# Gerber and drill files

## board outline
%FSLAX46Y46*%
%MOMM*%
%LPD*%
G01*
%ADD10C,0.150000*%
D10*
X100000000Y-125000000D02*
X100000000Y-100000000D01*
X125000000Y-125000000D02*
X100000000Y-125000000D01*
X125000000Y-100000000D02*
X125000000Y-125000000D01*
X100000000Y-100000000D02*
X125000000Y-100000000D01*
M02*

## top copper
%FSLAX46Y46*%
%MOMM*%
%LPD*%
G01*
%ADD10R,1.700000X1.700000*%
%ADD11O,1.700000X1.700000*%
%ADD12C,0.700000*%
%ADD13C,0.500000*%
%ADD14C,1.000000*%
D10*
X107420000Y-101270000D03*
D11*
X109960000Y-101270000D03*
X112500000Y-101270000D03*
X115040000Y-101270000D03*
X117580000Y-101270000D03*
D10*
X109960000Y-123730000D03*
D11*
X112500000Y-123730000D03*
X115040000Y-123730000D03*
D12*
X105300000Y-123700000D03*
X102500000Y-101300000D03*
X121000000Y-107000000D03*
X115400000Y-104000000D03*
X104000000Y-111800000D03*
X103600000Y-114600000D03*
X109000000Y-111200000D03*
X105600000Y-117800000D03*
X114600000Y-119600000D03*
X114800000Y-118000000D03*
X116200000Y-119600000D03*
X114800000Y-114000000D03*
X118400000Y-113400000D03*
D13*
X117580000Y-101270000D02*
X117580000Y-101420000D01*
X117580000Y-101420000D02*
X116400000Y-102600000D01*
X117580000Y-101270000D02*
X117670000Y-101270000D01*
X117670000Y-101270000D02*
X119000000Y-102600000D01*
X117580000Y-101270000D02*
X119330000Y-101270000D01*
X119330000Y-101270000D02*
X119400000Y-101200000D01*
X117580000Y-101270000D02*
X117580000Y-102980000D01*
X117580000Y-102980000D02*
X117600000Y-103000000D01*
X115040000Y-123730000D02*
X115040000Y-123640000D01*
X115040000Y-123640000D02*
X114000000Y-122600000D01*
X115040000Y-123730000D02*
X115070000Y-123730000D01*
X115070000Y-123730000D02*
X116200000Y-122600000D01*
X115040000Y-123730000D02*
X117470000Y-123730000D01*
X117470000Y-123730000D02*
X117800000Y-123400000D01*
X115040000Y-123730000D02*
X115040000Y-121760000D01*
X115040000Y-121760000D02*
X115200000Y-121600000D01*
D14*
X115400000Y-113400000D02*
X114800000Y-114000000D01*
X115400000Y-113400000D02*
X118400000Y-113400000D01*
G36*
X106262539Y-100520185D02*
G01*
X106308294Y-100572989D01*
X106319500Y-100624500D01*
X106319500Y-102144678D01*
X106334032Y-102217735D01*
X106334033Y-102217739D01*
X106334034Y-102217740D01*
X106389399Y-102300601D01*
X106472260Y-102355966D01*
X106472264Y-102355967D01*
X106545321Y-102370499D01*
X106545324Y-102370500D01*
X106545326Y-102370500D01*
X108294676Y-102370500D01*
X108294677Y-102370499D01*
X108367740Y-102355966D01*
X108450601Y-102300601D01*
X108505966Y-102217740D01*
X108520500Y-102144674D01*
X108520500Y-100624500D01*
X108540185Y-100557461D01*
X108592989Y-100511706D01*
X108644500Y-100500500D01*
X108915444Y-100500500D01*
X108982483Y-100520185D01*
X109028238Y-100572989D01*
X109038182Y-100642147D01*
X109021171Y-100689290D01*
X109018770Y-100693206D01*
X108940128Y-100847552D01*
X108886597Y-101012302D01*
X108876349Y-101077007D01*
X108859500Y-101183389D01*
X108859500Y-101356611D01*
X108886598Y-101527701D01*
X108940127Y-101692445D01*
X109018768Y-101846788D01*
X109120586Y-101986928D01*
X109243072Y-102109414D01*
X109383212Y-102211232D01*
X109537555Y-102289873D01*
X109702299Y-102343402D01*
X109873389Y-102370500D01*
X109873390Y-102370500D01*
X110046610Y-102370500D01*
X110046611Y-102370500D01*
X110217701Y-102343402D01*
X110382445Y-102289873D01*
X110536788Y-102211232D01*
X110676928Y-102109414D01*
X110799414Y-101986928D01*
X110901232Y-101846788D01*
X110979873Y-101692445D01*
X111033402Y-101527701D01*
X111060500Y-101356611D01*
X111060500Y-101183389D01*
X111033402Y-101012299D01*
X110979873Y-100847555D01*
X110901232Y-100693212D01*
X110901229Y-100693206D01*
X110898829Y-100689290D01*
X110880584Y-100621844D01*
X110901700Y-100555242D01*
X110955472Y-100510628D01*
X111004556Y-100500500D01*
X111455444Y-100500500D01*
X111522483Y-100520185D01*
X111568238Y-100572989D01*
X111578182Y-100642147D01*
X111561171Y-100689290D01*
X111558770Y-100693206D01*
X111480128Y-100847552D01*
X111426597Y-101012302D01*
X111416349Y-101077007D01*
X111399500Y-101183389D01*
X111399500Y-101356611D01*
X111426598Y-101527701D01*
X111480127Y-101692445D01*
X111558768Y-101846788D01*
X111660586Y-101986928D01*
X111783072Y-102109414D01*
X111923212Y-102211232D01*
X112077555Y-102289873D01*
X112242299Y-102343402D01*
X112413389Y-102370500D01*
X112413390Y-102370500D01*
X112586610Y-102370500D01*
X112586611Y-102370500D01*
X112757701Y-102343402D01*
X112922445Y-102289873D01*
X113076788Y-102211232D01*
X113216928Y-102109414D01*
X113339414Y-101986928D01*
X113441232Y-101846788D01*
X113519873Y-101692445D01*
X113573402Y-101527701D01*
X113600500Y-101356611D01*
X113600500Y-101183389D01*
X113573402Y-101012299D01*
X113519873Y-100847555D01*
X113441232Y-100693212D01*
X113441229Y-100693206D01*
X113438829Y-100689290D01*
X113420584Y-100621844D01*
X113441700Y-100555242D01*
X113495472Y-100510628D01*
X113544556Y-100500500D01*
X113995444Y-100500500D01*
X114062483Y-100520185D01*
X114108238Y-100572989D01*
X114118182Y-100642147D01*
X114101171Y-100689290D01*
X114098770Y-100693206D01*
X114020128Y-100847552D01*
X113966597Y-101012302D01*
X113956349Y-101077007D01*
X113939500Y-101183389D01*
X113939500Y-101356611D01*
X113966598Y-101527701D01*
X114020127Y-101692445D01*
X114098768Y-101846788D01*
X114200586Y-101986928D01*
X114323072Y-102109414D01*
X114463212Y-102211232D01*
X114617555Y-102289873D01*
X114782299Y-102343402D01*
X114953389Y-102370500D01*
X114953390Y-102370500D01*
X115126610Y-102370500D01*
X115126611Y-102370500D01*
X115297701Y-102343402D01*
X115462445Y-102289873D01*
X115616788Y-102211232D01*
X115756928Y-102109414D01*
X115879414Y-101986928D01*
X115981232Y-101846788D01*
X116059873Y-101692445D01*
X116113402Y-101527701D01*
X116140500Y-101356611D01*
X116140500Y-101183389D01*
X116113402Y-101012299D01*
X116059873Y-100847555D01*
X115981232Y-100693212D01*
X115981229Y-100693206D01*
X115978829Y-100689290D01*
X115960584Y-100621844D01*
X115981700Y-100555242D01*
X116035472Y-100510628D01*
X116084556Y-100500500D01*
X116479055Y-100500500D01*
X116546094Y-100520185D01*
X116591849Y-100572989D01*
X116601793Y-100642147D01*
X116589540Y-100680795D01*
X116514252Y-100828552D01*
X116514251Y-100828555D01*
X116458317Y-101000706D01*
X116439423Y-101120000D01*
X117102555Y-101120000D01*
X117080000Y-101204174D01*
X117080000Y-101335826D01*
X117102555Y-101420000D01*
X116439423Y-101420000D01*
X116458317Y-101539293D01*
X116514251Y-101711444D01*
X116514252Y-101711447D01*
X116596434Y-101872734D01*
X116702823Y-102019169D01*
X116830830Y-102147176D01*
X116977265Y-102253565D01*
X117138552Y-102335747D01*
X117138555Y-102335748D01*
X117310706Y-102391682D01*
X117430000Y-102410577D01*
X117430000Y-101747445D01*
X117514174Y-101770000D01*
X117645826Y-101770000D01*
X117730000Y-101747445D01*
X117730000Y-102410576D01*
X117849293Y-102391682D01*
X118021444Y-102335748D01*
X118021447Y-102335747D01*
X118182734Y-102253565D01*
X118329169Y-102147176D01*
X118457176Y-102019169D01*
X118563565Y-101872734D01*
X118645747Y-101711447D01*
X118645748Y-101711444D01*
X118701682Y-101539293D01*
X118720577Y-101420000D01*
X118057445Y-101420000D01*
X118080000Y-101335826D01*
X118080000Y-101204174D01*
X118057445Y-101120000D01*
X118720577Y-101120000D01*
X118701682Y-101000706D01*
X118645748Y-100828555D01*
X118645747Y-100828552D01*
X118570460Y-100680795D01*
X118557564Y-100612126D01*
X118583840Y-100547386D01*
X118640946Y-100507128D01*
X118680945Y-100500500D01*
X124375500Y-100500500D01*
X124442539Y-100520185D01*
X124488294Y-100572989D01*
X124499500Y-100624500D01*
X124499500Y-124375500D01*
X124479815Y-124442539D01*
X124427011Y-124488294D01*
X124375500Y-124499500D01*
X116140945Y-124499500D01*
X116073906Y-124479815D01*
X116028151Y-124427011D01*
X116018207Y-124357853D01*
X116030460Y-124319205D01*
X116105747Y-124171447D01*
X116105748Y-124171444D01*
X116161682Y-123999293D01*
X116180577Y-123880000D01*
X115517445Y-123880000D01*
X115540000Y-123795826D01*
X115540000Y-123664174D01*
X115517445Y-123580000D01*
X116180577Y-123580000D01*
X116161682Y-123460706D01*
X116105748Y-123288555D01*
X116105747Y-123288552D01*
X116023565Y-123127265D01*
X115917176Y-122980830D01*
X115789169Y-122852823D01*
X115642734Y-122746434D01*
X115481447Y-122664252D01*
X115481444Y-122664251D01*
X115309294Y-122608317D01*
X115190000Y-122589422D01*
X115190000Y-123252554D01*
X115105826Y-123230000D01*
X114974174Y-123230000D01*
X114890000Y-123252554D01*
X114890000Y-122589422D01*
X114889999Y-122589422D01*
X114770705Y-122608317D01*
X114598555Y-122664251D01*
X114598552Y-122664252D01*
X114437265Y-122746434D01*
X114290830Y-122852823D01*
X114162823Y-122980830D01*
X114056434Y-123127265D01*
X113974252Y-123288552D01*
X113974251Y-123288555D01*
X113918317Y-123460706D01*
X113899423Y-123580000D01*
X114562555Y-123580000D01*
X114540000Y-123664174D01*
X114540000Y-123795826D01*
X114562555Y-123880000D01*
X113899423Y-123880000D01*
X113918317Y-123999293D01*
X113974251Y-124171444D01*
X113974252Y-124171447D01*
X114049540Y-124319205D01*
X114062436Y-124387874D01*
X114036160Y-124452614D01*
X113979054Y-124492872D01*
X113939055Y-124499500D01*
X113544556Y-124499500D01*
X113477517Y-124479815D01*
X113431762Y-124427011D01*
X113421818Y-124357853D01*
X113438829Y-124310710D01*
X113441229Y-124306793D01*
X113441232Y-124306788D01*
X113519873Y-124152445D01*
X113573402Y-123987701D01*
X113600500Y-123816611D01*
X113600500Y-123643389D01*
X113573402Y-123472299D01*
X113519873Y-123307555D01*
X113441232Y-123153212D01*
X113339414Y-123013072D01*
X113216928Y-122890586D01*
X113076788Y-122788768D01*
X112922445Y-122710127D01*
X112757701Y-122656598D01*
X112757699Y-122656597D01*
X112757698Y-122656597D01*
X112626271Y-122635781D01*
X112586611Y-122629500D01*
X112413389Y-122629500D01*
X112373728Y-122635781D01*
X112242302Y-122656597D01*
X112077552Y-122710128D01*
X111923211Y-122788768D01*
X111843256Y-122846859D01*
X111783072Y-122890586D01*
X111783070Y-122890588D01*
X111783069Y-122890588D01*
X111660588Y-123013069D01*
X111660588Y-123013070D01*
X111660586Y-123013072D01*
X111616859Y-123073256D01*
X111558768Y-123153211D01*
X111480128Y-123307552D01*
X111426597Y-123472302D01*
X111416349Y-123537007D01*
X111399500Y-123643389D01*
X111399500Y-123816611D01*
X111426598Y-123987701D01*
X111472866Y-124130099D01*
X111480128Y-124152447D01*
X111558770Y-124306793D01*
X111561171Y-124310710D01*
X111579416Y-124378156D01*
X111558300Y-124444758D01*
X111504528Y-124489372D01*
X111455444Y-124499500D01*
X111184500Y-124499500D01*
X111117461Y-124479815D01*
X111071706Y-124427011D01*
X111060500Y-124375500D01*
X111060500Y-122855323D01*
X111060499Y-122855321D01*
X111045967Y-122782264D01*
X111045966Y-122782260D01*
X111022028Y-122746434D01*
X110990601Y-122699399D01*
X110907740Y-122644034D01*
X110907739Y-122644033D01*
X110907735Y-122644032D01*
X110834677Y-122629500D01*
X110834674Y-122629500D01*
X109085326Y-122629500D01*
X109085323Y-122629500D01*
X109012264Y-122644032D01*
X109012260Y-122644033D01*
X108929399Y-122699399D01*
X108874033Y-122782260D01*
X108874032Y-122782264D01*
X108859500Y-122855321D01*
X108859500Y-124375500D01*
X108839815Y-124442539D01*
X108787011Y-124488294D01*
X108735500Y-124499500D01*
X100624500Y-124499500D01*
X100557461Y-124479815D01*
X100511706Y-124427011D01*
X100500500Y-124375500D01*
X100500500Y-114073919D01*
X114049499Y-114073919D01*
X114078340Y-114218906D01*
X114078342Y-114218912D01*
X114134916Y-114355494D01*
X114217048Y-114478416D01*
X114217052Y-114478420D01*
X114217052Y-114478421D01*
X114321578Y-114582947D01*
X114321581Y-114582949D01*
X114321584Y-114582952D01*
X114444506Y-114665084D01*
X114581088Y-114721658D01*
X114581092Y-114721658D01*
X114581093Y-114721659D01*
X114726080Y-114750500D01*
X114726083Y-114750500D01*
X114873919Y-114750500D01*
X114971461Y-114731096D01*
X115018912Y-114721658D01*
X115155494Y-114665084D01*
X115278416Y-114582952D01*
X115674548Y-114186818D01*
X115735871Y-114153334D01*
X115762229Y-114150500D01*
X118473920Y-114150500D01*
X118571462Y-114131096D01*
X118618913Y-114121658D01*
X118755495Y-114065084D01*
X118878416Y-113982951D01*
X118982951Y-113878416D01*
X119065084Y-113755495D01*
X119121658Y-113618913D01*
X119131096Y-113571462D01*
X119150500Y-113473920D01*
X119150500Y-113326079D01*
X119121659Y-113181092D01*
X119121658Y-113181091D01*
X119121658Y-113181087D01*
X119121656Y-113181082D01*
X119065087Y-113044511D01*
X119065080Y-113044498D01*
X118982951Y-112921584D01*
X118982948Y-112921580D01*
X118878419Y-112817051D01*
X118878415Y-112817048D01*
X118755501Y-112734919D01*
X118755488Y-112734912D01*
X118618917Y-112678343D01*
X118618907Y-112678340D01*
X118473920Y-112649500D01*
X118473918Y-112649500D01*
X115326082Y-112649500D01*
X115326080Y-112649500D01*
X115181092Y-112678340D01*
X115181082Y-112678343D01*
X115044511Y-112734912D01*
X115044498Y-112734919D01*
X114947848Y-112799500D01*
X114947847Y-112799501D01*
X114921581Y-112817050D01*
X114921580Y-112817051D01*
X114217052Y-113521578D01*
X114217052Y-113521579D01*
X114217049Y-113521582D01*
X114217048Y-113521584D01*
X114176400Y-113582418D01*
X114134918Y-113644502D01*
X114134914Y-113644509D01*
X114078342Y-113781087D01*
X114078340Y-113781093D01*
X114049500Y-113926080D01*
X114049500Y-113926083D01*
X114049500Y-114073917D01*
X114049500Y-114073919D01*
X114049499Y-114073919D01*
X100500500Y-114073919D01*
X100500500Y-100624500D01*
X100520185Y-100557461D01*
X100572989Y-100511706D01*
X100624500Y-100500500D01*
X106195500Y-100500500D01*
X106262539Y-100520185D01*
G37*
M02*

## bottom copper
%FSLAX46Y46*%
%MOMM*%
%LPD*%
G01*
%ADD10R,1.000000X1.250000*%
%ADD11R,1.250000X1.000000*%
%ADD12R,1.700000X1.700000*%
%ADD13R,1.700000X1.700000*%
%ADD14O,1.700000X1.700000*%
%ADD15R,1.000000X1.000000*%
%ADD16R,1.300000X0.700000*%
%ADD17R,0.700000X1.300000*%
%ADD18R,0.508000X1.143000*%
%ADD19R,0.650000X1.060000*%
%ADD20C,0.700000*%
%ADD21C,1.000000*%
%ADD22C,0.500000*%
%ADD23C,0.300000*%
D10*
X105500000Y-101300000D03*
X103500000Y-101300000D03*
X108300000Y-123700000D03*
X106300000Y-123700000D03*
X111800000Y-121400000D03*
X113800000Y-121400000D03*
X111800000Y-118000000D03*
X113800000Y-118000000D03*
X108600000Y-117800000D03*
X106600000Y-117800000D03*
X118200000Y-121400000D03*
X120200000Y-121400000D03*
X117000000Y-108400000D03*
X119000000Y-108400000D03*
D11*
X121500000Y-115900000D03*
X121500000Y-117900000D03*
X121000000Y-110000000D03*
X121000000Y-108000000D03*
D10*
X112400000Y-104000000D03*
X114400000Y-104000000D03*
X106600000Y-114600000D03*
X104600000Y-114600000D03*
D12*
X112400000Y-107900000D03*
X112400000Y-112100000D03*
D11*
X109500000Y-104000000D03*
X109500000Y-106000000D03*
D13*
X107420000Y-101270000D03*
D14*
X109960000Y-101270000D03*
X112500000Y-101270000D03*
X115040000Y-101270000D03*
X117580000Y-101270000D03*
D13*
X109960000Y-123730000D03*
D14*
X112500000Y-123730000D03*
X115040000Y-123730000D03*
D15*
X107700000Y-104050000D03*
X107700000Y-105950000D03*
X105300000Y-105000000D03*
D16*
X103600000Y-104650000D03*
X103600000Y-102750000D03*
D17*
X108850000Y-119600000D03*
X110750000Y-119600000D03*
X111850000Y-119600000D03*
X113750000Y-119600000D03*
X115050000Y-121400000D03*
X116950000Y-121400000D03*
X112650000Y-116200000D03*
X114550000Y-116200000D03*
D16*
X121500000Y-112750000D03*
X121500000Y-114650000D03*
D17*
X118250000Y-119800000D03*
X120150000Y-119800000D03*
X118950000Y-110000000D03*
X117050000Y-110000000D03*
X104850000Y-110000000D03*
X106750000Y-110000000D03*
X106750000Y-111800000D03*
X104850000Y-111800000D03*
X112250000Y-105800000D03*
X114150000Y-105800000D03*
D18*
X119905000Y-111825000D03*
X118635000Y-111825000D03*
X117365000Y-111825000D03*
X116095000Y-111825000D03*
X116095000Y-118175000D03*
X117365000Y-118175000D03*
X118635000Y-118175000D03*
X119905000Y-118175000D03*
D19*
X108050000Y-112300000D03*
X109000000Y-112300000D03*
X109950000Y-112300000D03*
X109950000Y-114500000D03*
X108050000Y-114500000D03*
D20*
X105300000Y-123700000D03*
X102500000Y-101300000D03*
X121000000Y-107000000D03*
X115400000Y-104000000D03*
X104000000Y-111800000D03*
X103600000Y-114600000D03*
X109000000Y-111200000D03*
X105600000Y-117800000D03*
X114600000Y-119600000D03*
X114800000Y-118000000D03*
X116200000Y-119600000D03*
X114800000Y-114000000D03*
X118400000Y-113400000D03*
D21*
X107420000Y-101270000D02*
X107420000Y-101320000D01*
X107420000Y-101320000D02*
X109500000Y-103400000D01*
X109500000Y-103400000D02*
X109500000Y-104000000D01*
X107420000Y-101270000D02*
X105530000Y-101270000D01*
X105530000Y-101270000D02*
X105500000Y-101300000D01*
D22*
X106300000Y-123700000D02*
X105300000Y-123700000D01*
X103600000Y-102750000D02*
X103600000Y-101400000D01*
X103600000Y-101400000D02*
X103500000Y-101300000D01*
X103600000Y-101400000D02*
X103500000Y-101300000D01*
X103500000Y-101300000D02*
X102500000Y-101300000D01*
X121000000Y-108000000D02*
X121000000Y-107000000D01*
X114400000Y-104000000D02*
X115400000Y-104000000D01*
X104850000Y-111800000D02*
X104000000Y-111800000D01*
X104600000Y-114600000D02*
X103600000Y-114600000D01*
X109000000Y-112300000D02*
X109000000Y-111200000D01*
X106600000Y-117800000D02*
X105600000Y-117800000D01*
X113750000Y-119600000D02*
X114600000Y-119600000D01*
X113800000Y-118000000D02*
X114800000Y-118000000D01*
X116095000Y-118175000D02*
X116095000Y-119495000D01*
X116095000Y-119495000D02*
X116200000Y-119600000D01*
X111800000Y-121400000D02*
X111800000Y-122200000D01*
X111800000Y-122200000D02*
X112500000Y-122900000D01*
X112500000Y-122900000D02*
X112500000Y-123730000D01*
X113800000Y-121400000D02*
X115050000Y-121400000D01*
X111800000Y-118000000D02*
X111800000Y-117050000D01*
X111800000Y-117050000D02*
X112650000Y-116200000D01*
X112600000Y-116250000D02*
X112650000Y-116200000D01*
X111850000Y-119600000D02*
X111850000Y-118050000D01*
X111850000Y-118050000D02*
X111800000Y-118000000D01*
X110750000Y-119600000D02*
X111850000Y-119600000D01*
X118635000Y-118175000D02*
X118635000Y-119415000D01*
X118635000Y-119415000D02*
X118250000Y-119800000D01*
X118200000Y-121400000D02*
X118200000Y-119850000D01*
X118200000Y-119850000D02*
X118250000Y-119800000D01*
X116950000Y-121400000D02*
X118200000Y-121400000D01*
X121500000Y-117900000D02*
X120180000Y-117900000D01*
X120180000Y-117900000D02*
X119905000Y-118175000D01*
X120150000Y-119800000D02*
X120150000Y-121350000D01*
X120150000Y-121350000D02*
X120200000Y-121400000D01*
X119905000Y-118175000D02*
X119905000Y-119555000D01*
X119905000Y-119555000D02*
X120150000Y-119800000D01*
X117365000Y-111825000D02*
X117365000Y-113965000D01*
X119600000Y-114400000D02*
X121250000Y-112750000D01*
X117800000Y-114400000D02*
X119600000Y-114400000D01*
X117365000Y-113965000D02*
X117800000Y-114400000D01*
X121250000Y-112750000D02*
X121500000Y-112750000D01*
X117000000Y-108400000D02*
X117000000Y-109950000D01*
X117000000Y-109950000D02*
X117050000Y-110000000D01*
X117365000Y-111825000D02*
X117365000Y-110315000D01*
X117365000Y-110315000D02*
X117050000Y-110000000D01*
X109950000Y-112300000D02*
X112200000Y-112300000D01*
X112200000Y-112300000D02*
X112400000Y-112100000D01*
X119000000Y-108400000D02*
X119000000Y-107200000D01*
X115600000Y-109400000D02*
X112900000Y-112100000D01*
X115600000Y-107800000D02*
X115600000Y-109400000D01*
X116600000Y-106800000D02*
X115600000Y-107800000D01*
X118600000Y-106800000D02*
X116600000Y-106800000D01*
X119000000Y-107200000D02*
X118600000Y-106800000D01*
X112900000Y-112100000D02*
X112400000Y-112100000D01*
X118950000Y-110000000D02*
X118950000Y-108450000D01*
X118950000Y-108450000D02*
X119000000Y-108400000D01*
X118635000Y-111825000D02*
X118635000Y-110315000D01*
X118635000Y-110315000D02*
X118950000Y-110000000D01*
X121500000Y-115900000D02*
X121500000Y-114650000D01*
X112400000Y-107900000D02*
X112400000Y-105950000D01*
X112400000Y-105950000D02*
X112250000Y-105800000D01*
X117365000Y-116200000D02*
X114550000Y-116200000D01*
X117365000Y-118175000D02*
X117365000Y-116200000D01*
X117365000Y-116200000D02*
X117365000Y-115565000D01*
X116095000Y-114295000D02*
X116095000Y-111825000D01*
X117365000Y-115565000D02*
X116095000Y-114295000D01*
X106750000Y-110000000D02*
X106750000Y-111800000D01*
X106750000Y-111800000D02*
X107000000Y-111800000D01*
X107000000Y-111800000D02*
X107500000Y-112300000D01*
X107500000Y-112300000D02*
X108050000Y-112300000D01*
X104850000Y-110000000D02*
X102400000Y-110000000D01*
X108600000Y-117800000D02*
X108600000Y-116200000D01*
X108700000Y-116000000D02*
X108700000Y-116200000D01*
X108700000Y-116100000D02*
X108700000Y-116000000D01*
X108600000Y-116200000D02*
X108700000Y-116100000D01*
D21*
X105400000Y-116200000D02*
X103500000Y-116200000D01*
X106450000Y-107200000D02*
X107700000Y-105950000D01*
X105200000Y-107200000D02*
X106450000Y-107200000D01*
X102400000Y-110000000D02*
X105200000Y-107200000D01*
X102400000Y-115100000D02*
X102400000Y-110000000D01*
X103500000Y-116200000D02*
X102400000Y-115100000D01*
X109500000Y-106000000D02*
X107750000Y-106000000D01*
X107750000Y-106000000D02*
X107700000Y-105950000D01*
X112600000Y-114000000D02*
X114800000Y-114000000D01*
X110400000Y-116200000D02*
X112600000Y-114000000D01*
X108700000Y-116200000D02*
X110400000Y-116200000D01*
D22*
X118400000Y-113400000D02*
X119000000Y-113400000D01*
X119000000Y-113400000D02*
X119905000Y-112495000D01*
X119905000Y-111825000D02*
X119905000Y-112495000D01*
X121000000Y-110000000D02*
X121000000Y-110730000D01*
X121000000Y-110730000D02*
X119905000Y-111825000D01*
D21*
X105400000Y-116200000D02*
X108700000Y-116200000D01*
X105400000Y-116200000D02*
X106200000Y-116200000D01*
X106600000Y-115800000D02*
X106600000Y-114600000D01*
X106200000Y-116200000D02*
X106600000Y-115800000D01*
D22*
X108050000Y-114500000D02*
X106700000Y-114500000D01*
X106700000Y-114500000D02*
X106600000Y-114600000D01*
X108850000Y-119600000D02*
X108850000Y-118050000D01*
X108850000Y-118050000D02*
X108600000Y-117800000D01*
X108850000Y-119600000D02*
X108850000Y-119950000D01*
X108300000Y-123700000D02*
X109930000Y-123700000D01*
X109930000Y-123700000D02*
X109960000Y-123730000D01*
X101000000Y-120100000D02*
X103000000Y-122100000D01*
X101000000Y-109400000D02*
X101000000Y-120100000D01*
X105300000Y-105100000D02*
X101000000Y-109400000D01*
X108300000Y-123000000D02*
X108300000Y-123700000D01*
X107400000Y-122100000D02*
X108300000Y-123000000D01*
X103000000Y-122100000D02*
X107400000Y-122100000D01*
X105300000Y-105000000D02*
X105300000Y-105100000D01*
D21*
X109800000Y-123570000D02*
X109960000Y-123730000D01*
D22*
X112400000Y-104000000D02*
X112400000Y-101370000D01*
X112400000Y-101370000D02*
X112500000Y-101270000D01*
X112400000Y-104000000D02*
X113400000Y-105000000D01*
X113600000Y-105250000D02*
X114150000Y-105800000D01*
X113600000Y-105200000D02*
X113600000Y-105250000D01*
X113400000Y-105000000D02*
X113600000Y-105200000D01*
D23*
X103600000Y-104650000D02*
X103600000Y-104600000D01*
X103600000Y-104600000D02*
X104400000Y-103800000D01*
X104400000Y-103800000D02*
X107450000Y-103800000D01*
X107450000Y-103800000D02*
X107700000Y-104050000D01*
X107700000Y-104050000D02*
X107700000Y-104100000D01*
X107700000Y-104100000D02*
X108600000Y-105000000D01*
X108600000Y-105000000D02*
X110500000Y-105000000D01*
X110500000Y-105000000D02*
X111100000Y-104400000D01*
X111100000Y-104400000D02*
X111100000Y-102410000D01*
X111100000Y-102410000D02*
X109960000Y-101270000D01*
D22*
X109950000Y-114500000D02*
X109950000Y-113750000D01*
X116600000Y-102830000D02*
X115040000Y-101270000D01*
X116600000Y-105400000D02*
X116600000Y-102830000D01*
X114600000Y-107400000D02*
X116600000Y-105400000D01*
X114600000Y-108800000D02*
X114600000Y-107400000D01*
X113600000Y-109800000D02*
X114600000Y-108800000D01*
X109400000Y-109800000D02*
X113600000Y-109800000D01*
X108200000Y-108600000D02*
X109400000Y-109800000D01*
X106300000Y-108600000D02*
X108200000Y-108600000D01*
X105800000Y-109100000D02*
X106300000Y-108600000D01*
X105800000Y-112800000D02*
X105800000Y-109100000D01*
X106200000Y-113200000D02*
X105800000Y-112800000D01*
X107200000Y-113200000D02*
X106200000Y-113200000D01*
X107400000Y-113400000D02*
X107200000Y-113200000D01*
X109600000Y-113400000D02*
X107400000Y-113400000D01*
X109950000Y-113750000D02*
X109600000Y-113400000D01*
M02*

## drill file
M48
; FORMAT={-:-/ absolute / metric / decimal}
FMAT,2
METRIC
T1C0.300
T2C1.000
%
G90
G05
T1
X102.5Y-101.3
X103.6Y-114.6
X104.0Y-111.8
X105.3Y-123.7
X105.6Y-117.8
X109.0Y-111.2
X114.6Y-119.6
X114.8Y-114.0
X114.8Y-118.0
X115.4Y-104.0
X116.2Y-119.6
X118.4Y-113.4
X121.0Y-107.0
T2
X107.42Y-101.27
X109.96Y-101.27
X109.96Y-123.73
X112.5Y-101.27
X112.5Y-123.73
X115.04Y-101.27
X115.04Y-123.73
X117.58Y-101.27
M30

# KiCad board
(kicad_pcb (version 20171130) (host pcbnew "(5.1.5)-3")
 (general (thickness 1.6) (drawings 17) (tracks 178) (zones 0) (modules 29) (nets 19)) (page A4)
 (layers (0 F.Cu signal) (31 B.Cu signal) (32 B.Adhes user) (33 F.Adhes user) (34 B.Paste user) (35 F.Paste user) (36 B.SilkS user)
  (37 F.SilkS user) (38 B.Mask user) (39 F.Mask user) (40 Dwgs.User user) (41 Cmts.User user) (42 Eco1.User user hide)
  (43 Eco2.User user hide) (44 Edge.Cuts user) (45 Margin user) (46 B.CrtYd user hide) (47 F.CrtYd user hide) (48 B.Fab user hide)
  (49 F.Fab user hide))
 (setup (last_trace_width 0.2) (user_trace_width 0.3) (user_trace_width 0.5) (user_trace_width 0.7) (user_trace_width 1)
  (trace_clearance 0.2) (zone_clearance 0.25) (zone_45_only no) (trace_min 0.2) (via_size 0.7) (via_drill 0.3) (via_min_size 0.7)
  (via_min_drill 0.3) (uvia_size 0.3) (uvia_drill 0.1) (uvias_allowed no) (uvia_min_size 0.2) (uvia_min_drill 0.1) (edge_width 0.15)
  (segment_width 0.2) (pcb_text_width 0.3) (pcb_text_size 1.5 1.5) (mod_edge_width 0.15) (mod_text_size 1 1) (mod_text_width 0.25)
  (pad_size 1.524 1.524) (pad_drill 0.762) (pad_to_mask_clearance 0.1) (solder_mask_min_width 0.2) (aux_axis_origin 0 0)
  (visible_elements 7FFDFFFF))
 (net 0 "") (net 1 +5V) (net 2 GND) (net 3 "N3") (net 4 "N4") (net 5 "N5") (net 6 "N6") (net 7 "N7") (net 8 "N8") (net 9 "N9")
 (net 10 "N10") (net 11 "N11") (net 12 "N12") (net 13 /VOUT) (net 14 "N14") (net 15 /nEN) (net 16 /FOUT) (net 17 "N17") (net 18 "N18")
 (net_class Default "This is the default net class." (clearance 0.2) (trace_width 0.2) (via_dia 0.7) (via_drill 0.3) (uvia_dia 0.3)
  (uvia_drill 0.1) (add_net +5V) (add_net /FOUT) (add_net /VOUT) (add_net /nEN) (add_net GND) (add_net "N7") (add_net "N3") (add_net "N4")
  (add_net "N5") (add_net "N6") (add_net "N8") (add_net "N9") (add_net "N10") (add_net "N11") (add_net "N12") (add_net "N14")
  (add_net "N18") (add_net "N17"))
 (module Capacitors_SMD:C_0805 (layer B.Cu) (at 104.5 101.3 180)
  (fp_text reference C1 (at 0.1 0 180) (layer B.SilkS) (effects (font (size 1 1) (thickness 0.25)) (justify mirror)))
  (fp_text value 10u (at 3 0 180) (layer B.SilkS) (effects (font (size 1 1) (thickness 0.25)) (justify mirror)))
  (pad 1 smd rect (at -1 0 180) (size 1 1.25) (layers B.Cu B.Paste B.Mask) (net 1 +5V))
  (pad 2 smd rect (at 1 0 180) (size 1 1.25) (layers B.Cu B.Paste B.Mask) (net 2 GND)))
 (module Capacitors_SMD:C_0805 (layer B.Cu) (at 107.3 123.7 180)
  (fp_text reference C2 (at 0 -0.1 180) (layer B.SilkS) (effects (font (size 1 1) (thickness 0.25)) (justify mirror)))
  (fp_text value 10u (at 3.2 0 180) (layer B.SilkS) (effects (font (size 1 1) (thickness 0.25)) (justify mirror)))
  (pad 1 smd rect (at -1 0 180) (size 1 1.25) (layers B.Cu B.Paste B.Mask) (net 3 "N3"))
  (pad 2 smd rect (at 1 0 180) (size 1 1.25) (layers B.Cu B.Paste B.Mask) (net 2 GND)))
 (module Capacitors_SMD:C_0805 (layer B.Cu) (at 112.8 121.4)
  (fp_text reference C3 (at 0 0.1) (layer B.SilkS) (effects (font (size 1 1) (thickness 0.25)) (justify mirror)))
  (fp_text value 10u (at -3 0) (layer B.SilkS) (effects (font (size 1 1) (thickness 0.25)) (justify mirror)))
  (pad 1 smd rect (at -1 0) (size 1 1.25) (layers B.Cu B.Paste B.Mask) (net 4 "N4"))
  (pad 2 smd rect (at 1 0) (size 1 1.25) (layers B.Cu B.Paste B.Mask) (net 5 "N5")))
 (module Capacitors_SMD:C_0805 (layer B.Cu) (at 112.8 118)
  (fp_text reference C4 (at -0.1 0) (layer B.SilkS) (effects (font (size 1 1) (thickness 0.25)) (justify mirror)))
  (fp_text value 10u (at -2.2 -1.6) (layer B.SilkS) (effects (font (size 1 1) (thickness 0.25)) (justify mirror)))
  (pad 1 smd rect (at -1 0) (size 1 1.25) (layers B.Cu B.Paste B.Mask) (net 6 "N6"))
  (pad 2 smd rect (at 1 0) (size 1 1.25) (layers B.Cu B.Paste B.Mask) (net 2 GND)))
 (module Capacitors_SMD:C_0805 (layer B.Cu) (at 107.6 117.8 180)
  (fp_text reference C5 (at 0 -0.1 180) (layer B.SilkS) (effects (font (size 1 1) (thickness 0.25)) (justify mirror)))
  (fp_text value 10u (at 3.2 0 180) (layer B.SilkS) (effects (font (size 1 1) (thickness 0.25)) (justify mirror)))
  (pad 1 smd rect (at -1 0 180) (size 1 1.25) (layers B.Cu B.Paste B.Mask) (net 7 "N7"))
  (pad 2 smd rect (at 1 0 180) (size 1 1.25) (layers B.Cu B.Paste B.Mask) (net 2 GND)))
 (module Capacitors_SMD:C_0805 (layer B.Cu) (at 119.2 121.4)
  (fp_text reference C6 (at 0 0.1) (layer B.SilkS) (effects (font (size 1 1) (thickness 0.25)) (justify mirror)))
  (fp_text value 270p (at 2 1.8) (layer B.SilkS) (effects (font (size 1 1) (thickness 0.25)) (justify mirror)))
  (pad 1 smd rect (at -1 0) (size 1 1.25) (layers B.Cu B.Paste B.Mask) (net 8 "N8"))
  (pad 2 smd rect (at 1 0) (size 1 1.25) (layers B.Cu B.Paste B.Mask) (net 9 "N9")))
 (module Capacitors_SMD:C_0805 (layer B.Cu) (at 118 108.4)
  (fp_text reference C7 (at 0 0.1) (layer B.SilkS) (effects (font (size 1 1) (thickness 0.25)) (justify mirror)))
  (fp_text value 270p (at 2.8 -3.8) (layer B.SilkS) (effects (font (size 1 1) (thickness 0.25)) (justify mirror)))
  (pad 1 smd rect (at -1 0) (size 1 1.25) (layers B.Cu B.Paste B.Mask) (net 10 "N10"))
  (pad 2 smd rect (at 1 0) (size 1 1.25) (layers B.Cu B.Paste B.Mask) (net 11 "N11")))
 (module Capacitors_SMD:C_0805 (layer B.Cu) (at 121.5 116.9 270)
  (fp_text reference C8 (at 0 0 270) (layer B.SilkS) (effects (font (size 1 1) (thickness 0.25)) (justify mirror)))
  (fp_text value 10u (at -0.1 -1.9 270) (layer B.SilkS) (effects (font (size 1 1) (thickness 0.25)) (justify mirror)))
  (pad 1 smd rect (at -1 0 270) (size 1 1.25) (layers B.Cu B.Paste B.Mask) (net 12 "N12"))
  (pad 2 smd rect (at 1 0 270) (size 1 1.25) (layers B.Cu B.Paste B.Mask) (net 9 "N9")))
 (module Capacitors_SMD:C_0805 (layer B.Cu) (at 121 109 90)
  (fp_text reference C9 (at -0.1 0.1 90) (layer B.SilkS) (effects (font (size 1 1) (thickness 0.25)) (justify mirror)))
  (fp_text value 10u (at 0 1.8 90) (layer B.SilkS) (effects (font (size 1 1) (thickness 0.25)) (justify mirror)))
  (pad 1 smd rect (at -1 0 90) (size 1 1.25) (layers B.Cu B.Paste B.Mask) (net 7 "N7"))
  (pad 2 smd rect (at 1 0 90) (size 1 1.25) (layers B.Cu B.Paste B.Mask) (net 2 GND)))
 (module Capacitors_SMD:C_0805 (layer B.Cu) (at 113.4 104)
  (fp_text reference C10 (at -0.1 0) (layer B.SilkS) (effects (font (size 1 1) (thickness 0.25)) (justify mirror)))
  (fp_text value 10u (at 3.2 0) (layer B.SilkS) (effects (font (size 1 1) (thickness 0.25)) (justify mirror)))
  (pad 1 smd rect (at -1 0) (size 1 1.25) (layers B.Cu B.Paste B.Mask) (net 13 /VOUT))
  (pad 2 smd rect (at 1 0) (size 1 1.25) (layers B.Cu B.Paste B.Mask) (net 2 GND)))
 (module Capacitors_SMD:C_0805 (layer B.Cu) (at 105.6 114.6 180)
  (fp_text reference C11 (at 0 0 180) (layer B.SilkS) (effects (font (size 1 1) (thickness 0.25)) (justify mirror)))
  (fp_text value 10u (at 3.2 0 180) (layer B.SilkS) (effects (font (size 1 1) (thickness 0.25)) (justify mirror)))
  (pad 1 smd rect (at -1 0 180) (size 1 1.25) (layers B.Cu B.Paste B.Mask) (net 7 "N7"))
  (pad 2 smd rect (at 1 0 180) (size 1 1.25) (layers B.Cu B.Paste B.Mask) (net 2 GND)))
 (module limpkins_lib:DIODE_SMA (layer B.Cu) (at 112.4 110 270)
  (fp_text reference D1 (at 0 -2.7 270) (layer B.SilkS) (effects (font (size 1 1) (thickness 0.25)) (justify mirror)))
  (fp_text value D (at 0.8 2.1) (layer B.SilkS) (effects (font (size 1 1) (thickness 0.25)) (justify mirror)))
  (pad 1 smd rect (at -2.1 0 270) (size 1.7 1.7) (layers B.Cu B.Paste B.Mask) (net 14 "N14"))
  (pad 2 smd rect (at 2.1 0 270) (size 1.7 1.7) (layers B.Cu B.Paste B.Mask) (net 11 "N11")))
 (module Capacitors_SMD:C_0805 (layer B.Cu) (at 109.5 105 270)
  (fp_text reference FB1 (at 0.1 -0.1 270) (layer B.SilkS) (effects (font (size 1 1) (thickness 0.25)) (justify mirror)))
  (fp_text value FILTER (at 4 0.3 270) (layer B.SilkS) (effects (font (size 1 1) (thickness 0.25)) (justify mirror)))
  (pad 1 smd rect (at -1 0 270) (size 1 1.25) (layers B.Cu B.Paste B.Mask) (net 1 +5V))
  (pad 2 smd rect (at 1 0 270) (size 1 1.25) (layers B.Cu B.Paste B.Mask) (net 7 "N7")))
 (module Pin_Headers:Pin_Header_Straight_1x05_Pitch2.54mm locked (layer F.Cu) (at 107.42 101.27 90)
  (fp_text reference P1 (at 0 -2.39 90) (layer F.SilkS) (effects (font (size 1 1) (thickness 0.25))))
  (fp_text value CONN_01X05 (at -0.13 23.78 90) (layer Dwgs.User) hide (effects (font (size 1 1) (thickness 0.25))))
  (pad 1 thru_hole rect (at 0 0 90) (size 1.7 1.7) (drill 1) (layers *.Cu *.Mask) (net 1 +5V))
  (pad 2 thru_hole oval (at 0 2.54 90) (size 1.7 1.7) (drill 1) (layers *.Cu *.Mask) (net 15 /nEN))
  (pad 3 thru_hole oval (at 0 5.08 90) (size 1.7 1.7) (drill 1) (layers *.Cu *.Mask) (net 13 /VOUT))
  (pad 4 thru_hole oval (at 0 7.62 90) (size 1.7 1.7) (drill 1) (layers *.Cu *.Mask) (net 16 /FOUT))
  (pad 5 thru_hole oval (at 0 10.16 90) (size 1.7 1.7) (drill 1) (layers *.Cu *.Mask) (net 2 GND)))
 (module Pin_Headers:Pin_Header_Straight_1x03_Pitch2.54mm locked (layer F.Cu) (at 109.96 123.73 90)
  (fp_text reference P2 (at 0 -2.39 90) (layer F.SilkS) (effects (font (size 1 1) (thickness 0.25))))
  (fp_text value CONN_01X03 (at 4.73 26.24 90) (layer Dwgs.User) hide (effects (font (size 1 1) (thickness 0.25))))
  (pad 1 thru_hole rect (at 0 0 90) (size 1.7 1.7) (drill 1) (layers *.Cu *.Mask) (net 3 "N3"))
  (pad 2 thru_hole oval (at 0 2.54 90) (size 1.7 1.7) (drill 1) (layers *.Cu *.Mask) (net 4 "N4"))
  (pad 3 thru_hole oval (at 0 5.08 90) (size 1.7 1.7) (drill 1) (layers *.Cu *.Mask) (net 2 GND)))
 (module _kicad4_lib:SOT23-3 (layer B.Cu) (at 106.5 105 270)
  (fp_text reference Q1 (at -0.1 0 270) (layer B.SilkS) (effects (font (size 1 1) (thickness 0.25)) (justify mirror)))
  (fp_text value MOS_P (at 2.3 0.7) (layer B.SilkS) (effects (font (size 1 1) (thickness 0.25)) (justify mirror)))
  (pad 1 smd rect (at -0.95 -1.2 270) (size 1 1) (layers B.Cu B.Paste B.Mask) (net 15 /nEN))
  (pad 2 smd rect (at 0.95 -1.2 270) (size 1 1) (layers B.Cu B.Paste B.Mask) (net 7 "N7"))
  (pad 3 smd rect (at 0 1.2 270) (size 1 1) (layers B.Cu B.Paste B.Mask) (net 3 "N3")))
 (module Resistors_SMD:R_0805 (layer B.Cu) (at 103.6 103.7 90)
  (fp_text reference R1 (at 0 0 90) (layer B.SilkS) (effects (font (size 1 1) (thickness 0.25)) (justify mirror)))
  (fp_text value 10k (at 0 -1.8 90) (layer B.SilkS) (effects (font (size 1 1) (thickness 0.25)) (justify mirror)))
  (pad 1 smd rect (at -0.95 0 90) (size 0.7 1.3) (layers B.Cu B.Paste B.Mask) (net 15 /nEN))
  (pad 2 smd rect (at 0.95 0 90) (size 0.7 1.3) (layers B.Cu B.Paste B.Mask) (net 2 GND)))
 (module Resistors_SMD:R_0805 (layer B.Cu) (at 109.8 119.6)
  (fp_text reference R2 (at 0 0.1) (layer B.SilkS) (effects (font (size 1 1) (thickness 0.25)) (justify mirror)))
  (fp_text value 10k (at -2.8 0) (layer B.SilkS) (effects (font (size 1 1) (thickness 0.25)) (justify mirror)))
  (pad 1 smd rect (at -0.95 0) (size 0.7 1.3) (layers B.Cu B.Paste B.Mask) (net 7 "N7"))
  (pad 2 smd rect (at 0.95 0) (size 0.7 1.3) (layers B.Cu B.Paste B.Mask) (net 6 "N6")))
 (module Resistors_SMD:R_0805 (layer B.Cu) (at 112.8 119.6)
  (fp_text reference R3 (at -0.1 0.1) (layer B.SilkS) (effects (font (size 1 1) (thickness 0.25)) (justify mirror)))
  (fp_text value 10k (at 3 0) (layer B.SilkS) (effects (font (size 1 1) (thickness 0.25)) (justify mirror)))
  (pad 1 smd rect (at -0.95 0) (size 0.7 1.3) (layers B.Cu B.Paste B.Mask) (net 6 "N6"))
  (pad 2 smd rect (at 0.95 0) (size 0.7 1.3) (layers B.Cu B.Paste B.Mask) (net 2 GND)))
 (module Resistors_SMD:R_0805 (layer B.Cu) (at 116 121.4)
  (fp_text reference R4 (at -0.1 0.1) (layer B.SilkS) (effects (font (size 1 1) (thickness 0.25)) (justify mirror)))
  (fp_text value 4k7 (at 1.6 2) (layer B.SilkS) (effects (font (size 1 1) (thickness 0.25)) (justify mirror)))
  (pad 1 smd rect (at -0.95 0) (size 0.7 1.3) (layers B.Cu B.Paste B.Mask) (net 5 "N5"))
  (pad 2 smd rect (at 0.95 0) (size 0.7 1.3) (layers B.Cu B.Paste B.Mask) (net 8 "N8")))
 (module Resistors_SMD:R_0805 (layer B.Cu) (at 113.6 116.2)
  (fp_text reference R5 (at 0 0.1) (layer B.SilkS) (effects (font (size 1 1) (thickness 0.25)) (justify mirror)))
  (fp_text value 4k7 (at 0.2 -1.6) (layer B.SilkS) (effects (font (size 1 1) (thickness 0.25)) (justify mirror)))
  (pad 1 smd rect (at -0.95 0) (size 0.7 1.3) (layers B.Cu B.Paste B.Mask) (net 6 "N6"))
  (pad 2 smd rect (at 0.95 0) (size 0.7 1.3) (layers B.Cu B.Paste B.Mask) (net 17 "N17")))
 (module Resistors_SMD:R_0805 (layer B.Cu) (at 121.5 113.7 270)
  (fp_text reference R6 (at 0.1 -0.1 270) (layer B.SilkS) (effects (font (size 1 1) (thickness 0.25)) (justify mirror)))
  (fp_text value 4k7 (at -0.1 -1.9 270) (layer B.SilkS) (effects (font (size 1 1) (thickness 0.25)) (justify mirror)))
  (pad 1 smd rect (at -0.95 0 270) (size 0.7 1.3) (layers B.Cu B.Paste B.Mask) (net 10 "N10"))
  (pad 2 smd rect (at 0.95 0 270) (size 0.7 1.3) (layers B.Cu B.Paste B.Mask) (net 12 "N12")))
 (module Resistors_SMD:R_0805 (layer B.Cu) (at 119.2 119.8)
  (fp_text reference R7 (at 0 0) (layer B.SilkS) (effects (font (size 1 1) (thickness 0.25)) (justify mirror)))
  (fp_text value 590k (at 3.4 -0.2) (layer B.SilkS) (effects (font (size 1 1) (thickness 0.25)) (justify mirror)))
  (pad 1 smd rect (at -0.95 0) (size 0.7 1.3) (layers B.Cu B.Paste B.Mask) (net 8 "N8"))
  (pad 2 smd rect (at 0.95 0) (size 0.7 1.3) (layers B.Cu B.Paste B.Mask) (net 9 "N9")))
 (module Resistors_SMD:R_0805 (layer B.Cu) (at 118 110 180)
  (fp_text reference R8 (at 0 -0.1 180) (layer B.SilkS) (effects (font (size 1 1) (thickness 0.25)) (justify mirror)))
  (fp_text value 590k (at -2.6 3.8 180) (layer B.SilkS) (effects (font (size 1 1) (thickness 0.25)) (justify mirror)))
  (pad 1 smd rect (at -0.95 0 180) (size 0.7 1.3) (layers B.Cu B.Paste B.Mask) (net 11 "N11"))
  (pad 2 smd rect (at 0.95 0 180) (size 0.7 1.3) (layers B.Cu B.Paste B.Mask) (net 10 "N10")))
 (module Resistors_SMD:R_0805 (layer B.Cu) (at 105.8 110)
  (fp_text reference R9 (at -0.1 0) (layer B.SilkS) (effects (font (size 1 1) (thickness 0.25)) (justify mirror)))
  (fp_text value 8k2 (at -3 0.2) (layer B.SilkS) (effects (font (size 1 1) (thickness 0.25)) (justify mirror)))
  (pad 1 smd rect (at -0.95 0) (size 0.7 1.3) (layers B.Cu B.Paste B.Mask) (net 7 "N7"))
  (pad 2 smd rect (at 0.95 0) (size 0.7 1.3) (layers B.Cu B.Paste B.Mask) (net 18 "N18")))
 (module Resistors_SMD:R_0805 (layer B.Cu) (at 105.8 111.8 180)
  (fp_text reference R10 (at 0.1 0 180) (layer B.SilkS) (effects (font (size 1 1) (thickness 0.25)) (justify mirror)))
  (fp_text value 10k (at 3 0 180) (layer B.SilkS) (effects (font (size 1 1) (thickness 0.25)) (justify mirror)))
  (pad 1 smd rect (at -0.95 0 180) (size 0.7 1.3) (layers B.Cu B.Paste B.Mask) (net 18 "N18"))
  (pad 2 smd rect (at 0.95 0 180) (size 0.7 1.3) (layers B.Cu B.Paste B.Mask) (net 2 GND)))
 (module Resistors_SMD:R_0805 (layer B.Cu) (at 113.2 105.8)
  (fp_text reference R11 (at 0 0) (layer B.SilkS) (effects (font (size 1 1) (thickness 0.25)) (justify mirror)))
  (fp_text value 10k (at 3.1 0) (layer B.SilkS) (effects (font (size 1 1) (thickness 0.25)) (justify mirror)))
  (pad 1 smd rect (at -0.95 0) (size 0.7 1.3) (layers B.Cu B.Paste B.Mask) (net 14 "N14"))
  (pad 2 smd rect (at 0.95 0) (size 0.7 1.3) (layers B.Cu B.Paste B.Mask) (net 13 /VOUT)))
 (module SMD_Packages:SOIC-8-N (layer B.Cu) (at 118 115 180)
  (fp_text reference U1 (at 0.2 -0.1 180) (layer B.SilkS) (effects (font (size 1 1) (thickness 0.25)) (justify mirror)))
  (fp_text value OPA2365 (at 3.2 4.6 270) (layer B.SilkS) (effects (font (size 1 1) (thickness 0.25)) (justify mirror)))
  (pad 8 smd rect (at -1.905 3.175 180) (size 0.508 1.143) (layers B.Cu B.Paste B.Mask) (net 7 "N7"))
  (pad 7 smd rect (at -0.635 3.175 180) (size 0.508 1.143) (layers B.Cu B.Paste B.Mask) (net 11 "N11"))
  (pad 6 smd rect (at 0.635 3.175 180) (size 0.508 1.143) (layers B.Cu B.Paste B.Mask) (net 10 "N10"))
  (pad 5 smd rect (at 1.905 3.175 180) (size 0.508 1.143) (layers B.Cu B.Paste B.Mask) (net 17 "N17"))
  (pad 4 smd rect (at 1.905 -3.175 180) (size 0.508 1.143) (layers B.Cu B.Paste B.Mask) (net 2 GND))
  (pad 3 smd rect (at 0.635 -3.175 180) (size 0.508 1.143) (layers B.Cu B.Paste B.Mask) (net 17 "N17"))
  (pad 2 smd rect (at -0.635 -3.175 180) (size 0.508 1.143) (layers B.Cu B.Paste B.Mask) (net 8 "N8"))
  (pad 1 smd rect (at -1.905 -3.175 180) (size 0.508 1.143) (layers B.Cu B.Paste B.Mask) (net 9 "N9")))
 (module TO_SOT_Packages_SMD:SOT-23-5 (layer B.Cu) (at 109 113.4 270)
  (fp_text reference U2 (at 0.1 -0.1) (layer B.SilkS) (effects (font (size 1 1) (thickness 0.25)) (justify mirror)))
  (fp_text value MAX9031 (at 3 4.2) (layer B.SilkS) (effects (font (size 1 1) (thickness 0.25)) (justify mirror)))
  (pad 1 smd rect (at -1.1 0.95 270) (size 1.06 0.65) (layers B.Cu B.Paste B.Mask) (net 18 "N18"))
  (pad 2 smd rect (at -1.1 0 270) (size 1.06 0.65) (layers B.Cu B.Paste B.Mask) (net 2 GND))
  (pad 3 smd rect (at -1.1 -0.95 270) (size 1.06 0.65) (layers B.Cu B.Paste B.Mask) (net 11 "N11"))
  (pad 4 smd rect (at 1.1 -0.95 270) (size 1.06 0.65) (layers B.Cu B.Paste B.Mask) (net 16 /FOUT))
  (pad 5 smd rect (at 1.1 0.95 270) (size 1.06 0.65) (layers B.Cu B.Paste B.Mask) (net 7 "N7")))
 (gr_line (start 100 125) (end 100 100) (angle 90) (layer Edge.Cuts) (width 0.15))
 (gr_line (start 125 125) (end 100 125) (angle 90) (layer Edge.Cuts) (width 0.15))
 (gr_line (start 125 100) (end 125 125) (angle 90) (layer Edge.Cuts) (width 0.15))
 (gr_line (start 100 100) (end 125 100) (angle 90) (layer Edge.Cuts) (width 0.15))
 (segment (start 107.42 101.27) (end 107.42 101.32) (width 1) (layer B.Cu) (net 1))
 (segment (start 107.42 101.32) (end 109.5 103.4) (width 1) (layer B.Cu) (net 1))
 (segment (start 109.5 103.4) (end 109.5 104) (width 1) (layer B.Cu) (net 1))
 (segment (start 107.42 101.27) (end 105.53 101.27) (width 1) (layer B.Cu) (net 1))
 (segment (start 105.53 101.27) (end 105.5 101.3) (width 1) (layer B.Cu) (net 1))
 (segment (start 106.3 123.7) (end 105.3 123.7) (width 0.5) (layer B.Cu) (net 2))
 (via (at 105.3 123.7) (size 0.7) (drill 0.3) (layers F.Cu B.Cu) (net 2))
 (segment (start 103.6 102.75) (end 103.6 101.4) (width 0.5) (layer B.Cu) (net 2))
 (segment (start 103.6 101.4) (end 103.5 101.3) (width 0.5) (layer B.Cu) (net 2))
 (segment (start 103.6 101.4) (end 103.5 101.3) (width 0.5) (layer B.Cu) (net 2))
 (segment (start 103.5 101.3) (end 102.5 101.3) (width 0.5) (layer B.Cu) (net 2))
 (via (at 102.5 101.3) (size 0.7) (drill 0.3) (layers F.Cu B.Cu) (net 2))
 (segment (start 117.58 101.27) (end 117.58 101.42) (width 0.5) (layer F.Cu) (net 2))
 (segment (start 117.58 101.42) (end 116.4 102.6) (width 0.5) (layer F.Cu) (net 2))
 (segment (start 117.58 101.27) (end 117.67 101.27) (width 0.5) (layer F.Cu) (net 2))
 (segment (start 117.67 101.27) (end 119 102.6) (width 0.5) (layer F.Cu) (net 2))
 (segment (start 117.58 101.27) (end 119.33 101.27) (width 0.5) (layer F.Cu) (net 2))
 (segment (start 119.33 101.27) (end 119.4 101.2) (width 0.5) (layer F.Cu) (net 2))
 (segment (start 117.58 101.27) (end 117.58 102.98) (width 0.5) (layer F.Cu) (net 2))
 (segment (start 117.58 102.98) (end 117.6 103) (width 0.5) (layer F.Cu) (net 2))
 (segment (start 115.04 123.73) (end 115.04 123.64) (width 0.5) (layer F.Cu) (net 2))
 (segment (start 115.04 123.64) (end 114 122.6) (width 0.5) (layer F.Cu) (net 2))
 (segment (start 115.04 123.73) (end 115.07 123.73) (width 0.5) (layer F.Cu) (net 2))
 (segment (start 115.07 123.73) (end 116.2 122.6) (width 0.5) (layer F.Cu) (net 2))
 (segment (start 115.04 123.73) (end 117.47 123.73) (width 0.5) (layer F.Cu) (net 2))
 (segment (start 117.47 123.73) (end 117.8 123.4) (width 0.5) (layer F.Cu) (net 2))
 (segment (start 115.04 123.73) (end 115.04 121.76) (width 0.5) (layer F.Cu) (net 2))
 (segment (start 115.04 121.76) (end 115.2 121.6) (width 0.5) (layer F.Cu) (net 2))
 (segment (start 121 108) (end 121 107) (width 0.5) (layer B.Cu) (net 2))
 (via (at 121 107) (size 0.7) (drill 0.3) (layers F.Cu B.Cu) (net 2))
 (segment (start 114.4 104) (end 115.4 104) (width 0.5) (layer B.Cu) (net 2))
 (via (at 115.4 104) (size 0.7) (drill 0.3) (layers F.Cu B.Cu) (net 2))
 (segment (start 104.85 111.8) (end 104 111.8) (width 0.5) (layer B.Cu) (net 2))
 (via (at 104 111.8) (size 0.7) (drill 0.3) (layers F.Cu B.Cu) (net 2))
 (segment (start 104.6 114.6) (end 103.6 114.6) (width 0.5) (layer B.Cu) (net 2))
 (via (at 103.6 114.6) (size 0.7) (drill 0.3) (layers F.Cu B.Cu) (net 2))
 (segment (start 109 112.3) (end 109 111.2) (width 0.5) (layer B.Cu) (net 2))
 (via (at 109 111.2) (size 0.7) (drill 0.3) (layers F.Cu B.Cu) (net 2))
 (segment (start 106.6 117.8) (end 105.6 117.8) (width 0.5) (layer B.Cu) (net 2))
 (via (at 105.6 117.8) (size 0.7) (drill 0.3) (layers F.Cu B.Cu) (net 2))
 (segment (start 113.75 119.6) (end 114.6 119.6) (width 0.5) (layer B.Cu) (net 2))
 (via (at 114.6 119.6) (size 0.7) (drill 0.3) (layers F.Cu B.Cu) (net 2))
 (segment (start 113.8 118) (end 114.8 118) (width 0.5) (layer B.Cu) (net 2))
 (via (at 114.8 118) (size 0.7) (drill 0.3) (layers F.Cu B.Cu) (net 2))
 (segment (start 116.095 118.175) (end 116.095 119.495) (width 0.5) (layer B.Cu) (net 2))
 (via (at 116.2 119.6) (size 0.7) (drill 0.3) (layers F.Cu B.Cu) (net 2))
 (segment (start 116.095 119.495) (end 116.2 119.6) (width 0.5) (layer B.Cu) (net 2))
 (segment (start 111.8 121.4) (end 111.8 122.2) (width 0.5) (layer B.Cu) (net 4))
 (segment (start 111.8 122.2) (end 112.5 122.9) (width 0.5) (layer B.Cu) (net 4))
 (segment (start 112.5 122.9) (end 112.5 123.73) (width 0.5) (layer B.Cu) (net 4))
 (segment (start 113.8 121.4) (end 115.05 121.4) (width 0.5) (layer B.Cu) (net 5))
 (segment (start 111.8 118) (end 111.8 117.05) (width 0.5) (layer B.Cu) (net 6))
 (segment (start 111.8 117.05) (end 112.65 116.2) (width 0.5) (layer B.Cu) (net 6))
 (segment (start 112.6 116.25) (end 112.65 116.2) (width 0.5) (layer B.Cu) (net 6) (status 30))
 (segment (start 111.85 119.6) (end 111.85 118.05) (width 0.5) (layer B.Cu) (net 6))
 (segment (start 111.85 118.05) (end 111.8 118) (width 0.5) (layer B.Cu) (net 6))
 (segment (start 110.75 119.6) (end 111.85 119.6) (width 0.5) (layer B.Cu) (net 6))
 (segment (start 118.635 118.175) (end 118.635 119.415) (width 0.5) (layer B.Cu) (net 8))
 (segment (start 118.635 119.415) (end 118.25 119.8) (width 0.5) (layer B.Cu) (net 8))
 (segment (start 118.2 121.4) (end 118.2 119.85) (width 0.5) (layer B.Cu) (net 8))
 (segment (start 118.2 119.85) (end 118.25 119.8) (width 0.5) (layer B.Cu) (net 8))
 (segment (start 116.95 121.4) (end 118.2 121.4) (width 0.5) (layer B.Cu) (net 8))
 (segment (start 121.5 117.9) (end 120.18 117.9) (width 0.5) (layer B.Cu) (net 9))
 (segment (start 120.18 117.9) (end 119.905 118.175) (width 0.5) (layer B.Cu) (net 9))
 (segment (start 120.15 119.8) (end 120.15 121.35) (width 0.5) (layer B.Cu) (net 9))
 (segment (start 120.15 121.35) (end 120.2 121.4) (width 0.5) (layer B.Cu) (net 9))
 (segment (start 119.905 118.175) (end 119.905 119.555) (width 0.5) (layer B.Cu) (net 9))
 (segment (start 119.905 119.555) (end 120.15 119.8) (width 0.5) (layer B.Cu) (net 9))
 (segment (start 117.365 111.825) (end 117.365 113.965) (width 0.5) (layer B.Cu) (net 10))
 (segment (start 119.6 114.4) (end 121.25 112.75) (width 0.5) (layer B.Cu) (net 10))
 (segment (start 117.8 114.4) (end 119.6 114.4) (width 0.5) (layer B.Cu) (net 10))
 (segment (start 117.365 113.965) (end 117.8 114.4) (width 0.5) (layer B.Cu) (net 10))
 (segment (start 121.25 112.75) (end 121.5 112.75) (width 0.5) (layer B.Cu) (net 10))
 (segment (start 117 108.4) (end 117 109.95) (width 0.5) (layer B.Cu) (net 10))
 (segment (start 117 109.95) (end 117.05 110) (width 0.5) (layer B.Cu) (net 10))
 (segment (start 117.365 111.825) (end 117.365 110.315) (width 0.5) (layer B.Cu) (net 10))
 (segment (start 117.365 110.315) (end 117.05 110) (width 0.5) (layer B.Cu) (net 10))
 (segment (start 109.95 112.3) (end 112.2 112.3) (width 0.5) (layer B.Cu) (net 11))
 (segment (start 112.2 112.3) (end 112.4 112.1) (width 0.5) (layer B.Cu) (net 11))
 (segment (start 119 108.4) (end 119 107.2) (width 0.5) (layer B.Cu) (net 11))
 (segment (start 115.6 109.4) (end 112.9 112.1) (width 0.5) (layer B.Cu) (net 11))
 (segment (start 115.6 107.8) (end 115.6 109.4) (width 0.5) (layer B.Cu) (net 11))
 (segment (start 116.6 106.8) (end 115.6 107.8) (width 0.5) (layer B.Cu) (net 11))
 (segment (start 118.6 106.8) (end 116.6 106.8) (width 0.5) (layer B.Cu) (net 11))
 (segment (start 119 107.2) (end 118.6 106.8) (width 0.5) (layer B.Cu) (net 11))
 (segment (start 112.9 112.1) (end 112.4 112.1) (width 0.5) (layer B.Cu) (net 11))
 (segment (start 118.95 110) (end 118.95 108.45) (width 0.5) (layer B.Cu) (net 11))
 (segment (start 118.95 108.45) (end 119 108.4) (width 0.5) (layer B.Cu) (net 11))
 (segment (start 118.635 111.825) (end 118.635 110.315) (width 0.5) (layer B.Cu) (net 11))
 (segment (start 118.635 110.315) (end 118.95 110) (width 0.5) (layer B.Cu) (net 11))
 (segment (start 121.5 115.9) (end 121.5 114.65) (width 0.5) (layer B.Cu) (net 12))
 (segment (start 112.4 107.9) (end 112.4 105.95) (width 0.5) (layer B.Cu) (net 14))
 (segment (start 112.4 105.95) (end 112.25 105.8) (width 0.5) (layer B.Cu) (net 14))
 (segment (start 117.365 116.2) (end 114.55 116.2) (width 0.5) (layer B.Cu) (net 17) (status 20))
 (segment (start 117.365 118.175) (end 117.365 116.2) (width 0.5) (layer B.Cu) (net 17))
 (segment (start 117.365 116.2) (end 117.365 115.565) (width 0.5) (layer B.Cu) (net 17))
 (segment (start 116.095 114.295) (end 116.095 111.825) (width 0.5) (layer B.Cu) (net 17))
 (segment (start 117.365 115.565) (end 116.095 114.295) (width 0.5) (layer B.Cu) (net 17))
 (segment (start 106.75 110) (end 106.75 111.8) (width 0.5) (layer B.Cu) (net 18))
 (segment (start 106.75 111.8) (end 107 111.8) (width 0.5) (layer B.Cu) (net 18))
 (segment (start 107 111.8) (end 107.5 112.3) (width 0.5) (layer B.Cu) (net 18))
 (segment (start 107.5 112.3) (end 108.05 112.3) (width 0.5) (layer B.Cu) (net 18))
 (segment (start 104.85 110) (end 102.4 110) (width 0.5) (layer B.Cu) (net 7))
 (segment (start 108.6 117.8) (end 108.6 116.2) (width 0.5) (layer B.Cu) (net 7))
 (segment (start 108.7 116) (end 108.7 116.2) (width 0.5) (layer B.Cu) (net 7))
 (segment (start 108.7 116.1) (end 108.7 116) (width 0.5) (layer B.Cu) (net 7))
 (segment (start 108.6 116.2) (end 108.7 116.1) (width 0.5) (layer B.Cu) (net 7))
 (segment (start 105.4 116.2) (end 103.5 116.2) (width 1) (layer B.Cu) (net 7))
 (segment (start 106.45 107.2) (end 107.7 105.95) (width 1) (layer B.Cu) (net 7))
 (segment (start 105.2 107.2) (end 106.45 107.2) (width 1) (layer B.Cu) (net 7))
 (segment (start 102.4 110) (end 105.2 107.2) (width 1) (layer B.Cu) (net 7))
 (segment (start 102.4 115.1) (end 102.4 110) (width 1) (layer B.Cu) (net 7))
 (segment (start 103.5 116.2) (end 102.4 115.1) (width 1) (layer B.Cu) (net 7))
 (segment (start 109.5 106) (end 107.75 106) (width 1) (layer B.Cu) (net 7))
 (segment (start 107.75 106) (end 107.7 105.95) (width 1) (layer B.Cu) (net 7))
 (via (at 114.8 114) (size 0.7) (drill 0.3) (layers F.Cu B.Cu) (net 7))
 (segment (start 112.6 114) (end 114.8 114) (width 1) (layer B.Cu) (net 7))
 (segment (start 110.4 116.2) (end 112.6 114) (width 1) (layer B.Cu) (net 7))
 (segment (start 108.7 116.2) (end 110.4 116.2) (width 1) (layer B.Cu) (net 7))
 (segment (start 115.4 113.4) (end 114.8 114) (width 1) (layer F.Cu) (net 7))
 (segment (start 115.4 113.4) (end 118.4 113.4) (width 1) (layer F.Cu) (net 7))
 (via (at 118.4 113.4) (size 0.7) (drill 0.3) (layers F.Cu B.Cu) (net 7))
 (segment (start 118.4 113.4) (end 119 113.4) (width 0.5) (layer B.Cu) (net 7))
 (segment (start 119 113.4) (end 119.905 112.495) (width 0.5) (layer B.Cu) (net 7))
 (segment (start 119.905 111.825) (end 119.905 112.495) (width 0.5) (layer B.Cu) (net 7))
 (segment (start 121 110) (end 121 110.73) (width 0.5) (layer B.Cu) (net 7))
 (segment (start 121 110.73) (end 119.905 111.825) (width 0.5) (layer B.Cu) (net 7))
 (segment (start 105.4 116.2) (end 108.7 116.2) (width 1) (layer B.Cu) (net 7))
 (segment (start 105.4 116.2) (end 106.2 116.2) (width 1) (layer B.Cu) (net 7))
 (segment (start 106.6 115.8) (end 106.6 114.6) (width 1) (layer B.Cu) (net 7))
 (segment (start 106.2 116.2) (end 106.6 115.8) (width 1) (layer B.Cu) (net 7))
 (segment (start 108.05 114.5) (end 106.7 114.5) (width 0.5) (layer B.Cu) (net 7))
 (segment (start 106.7 114.5) (end 106.6 114.6) (width 0.5) (layer B.Cu) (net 7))
 (segment (start 108.85 119.6) (end 108.85 118.05) (width 0.5) (layer B.Cu) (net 7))
 (segment (start 108.85 118.05) (end 108.6 117.8) (width 0.5) (layer B.Cu) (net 7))
 (segment (start 108.85 119.6) (end 108.85 119.95) (width 0.5) (layer B.Cu) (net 7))
 (segment (start 108.3 123.7) (end 109.93 123.7) (width 0.5) (layer B.Cu) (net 3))
 (segment (start 109.93 123.7) (end 109.96 123.73) (width 0.5) (layer B.Cu) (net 3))
 (segment (start 101 120.1) (end 103 122.1) (width 0.5) (layer B.Cu) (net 3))
 (segment (start 101 109.4) (end 101 120.1) (width 0.5) (layer B.Cu) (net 3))
 (segment (start 105.3 105.1) (end 101 109.4) (width 0.5) (layer B.Cu) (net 3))
 (segment (start 108.3 123) (end 108.3 123.7) (width 0.5) (layer B.Cu) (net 3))
 (segment (start 107.4 122.1) (end 108.3 123) (width 0.5) (layer B.Cu) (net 3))
 (segment (start 103 122.1) (end 107.4 122.1) (width 0.5) (layer B.Cu) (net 3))
 (segment (start 105.3 105) (end 105.3 105.1) (width 0.5) (layer B.Cu) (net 3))
 (segment (start 109.8 123.57) (end 109.96 123.73) (width 1) (layer B.Cu) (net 3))
 (segment (start 112.4 104) (end 112.4 101.37) (width 0.5) (layer B.Cu) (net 13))
 (segment (start 112.4 101.37) (end 112.5 101.27) (width 0.5) (layer B.Cu) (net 13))
 (segment (start 112.4 104) (end 113.4 105) (width 0.5) (layer B.Cu) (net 13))
 (segment (start 113.6 105.25) (end 114.15 105.8) (width 0.5) (layer B.Cu) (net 13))
 (segment (start 113.6 105.2) (end 113.6 105.25) (width 0.5) (layer B.Cu) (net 13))
 (segment (start 113.4 105) (end 113.6 105.2) (width 0.5) (layer B.Cu) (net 13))
 (segment (start 103.6 104.65) (end 103.6 104.6) (width 0.3) (layer B.Cu) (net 15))
 (segment (start 103.6 104.6) (end 104.4 103.8) (width 0.3) (layer B.Cu) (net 15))
 (segment (start 104.4 103.8) (end 107.45 103.8) (width 0.3) (layer B.Cu) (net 15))
 (segment (start 107.45 103.8) (end 107.7 104.05) (width 0.3) (layer B.Cu) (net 15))
 (segment (start 107.7 104.05) (end 107.7 104.1) (width 0.3) (layer B.Cu) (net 15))
 (segment (start 107.7 104.1) (end 108.6 105) (width 0.3) (layer B.Cu) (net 15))
 (segment (start 108.6 105) (end 110.5 105) (width 0.3) (layer B.Cu) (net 15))
 (segment (start 110.5 105) (end 111.1 104.4) (width 0.3) (layer B.Cu) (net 15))
 (segment (start 111.1 104.4) (end 111.1 102.41) (width 0.3) (layer B.Cu) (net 15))
 (segment (start 111.1 102.41) (end 109.96 101.27) (width 0.3) (layer B.Cu) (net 15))
 (segment (start 109.95 114.5) (end 109.95 113.75) (width 0.5) (layer B.Cu) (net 16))
 (segment (start 116.6 102.83) (end 115.04 101.27) (width 0.5) (layer B.Cu) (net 16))
 (segment (start 116.6 105.4) (end 116.6 102.83) (width 0.5) (layer B.Cu) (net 16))
 (segment (start 114.6 107.4) (end 116.6 105.4) (width 0.5) (layer B.Cu) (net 16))
 (segment (start 114.6 108.8) (end 114.6 107.4) (width 0.5) (layer B.Cu) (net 16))
 (segment (start 113.6 109.8) (end 114.6 108.8) (width 0.5) (layer B.Cu) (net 16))
 (segment (start 109.4 109.8) (end 113.6 109.8) (width 0.5) (layer B.Cu) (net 16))
 (segment (start 108.2 108.6) (end 109.4 109.8) (width 0.5) (layer B.Cu) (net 16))
 (segment (start 106.3 108.6) (end 108.2 108.6) (width 0.5) (layer B.Cu) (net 16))
 (segment (start 105.8 109.1) (end 106.3 108.6) (width 0.5) (layer B.Cu) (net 16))
 (segment (start 105.8 112.8) (end 105.8 109.1) (width 0.5) (layer B.Cu) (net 16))
 (segment (start 106.2 113.2) (end 105.8 112.8) (width 0.5) (layer B.Cu) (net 16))
 (segment (start 107.2 113.2) (end 106.2 113.2) (width 0.5) (layer B.Cu) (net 16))
 (segment (start 107.4 113.4) (end 107.2 113.2) (width 0.5) (layer B.Cu) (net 16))
 (segment (start 109.6 113.4) (end 107.4 113.4) (width 0.5) (layer B.Cu) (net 16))
 (segment (start 109.95 113.75) (end 109.6 113.4) (width 0.5) (layer B.Cu) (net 16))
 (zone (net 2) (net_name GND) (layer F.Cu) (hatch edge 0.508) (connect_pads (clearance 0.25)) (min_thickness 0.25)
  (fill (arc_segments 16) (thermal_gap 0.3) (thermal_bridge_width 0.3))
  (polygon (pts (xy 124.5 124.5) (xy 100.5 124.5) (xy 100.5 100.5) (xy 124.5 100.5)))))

